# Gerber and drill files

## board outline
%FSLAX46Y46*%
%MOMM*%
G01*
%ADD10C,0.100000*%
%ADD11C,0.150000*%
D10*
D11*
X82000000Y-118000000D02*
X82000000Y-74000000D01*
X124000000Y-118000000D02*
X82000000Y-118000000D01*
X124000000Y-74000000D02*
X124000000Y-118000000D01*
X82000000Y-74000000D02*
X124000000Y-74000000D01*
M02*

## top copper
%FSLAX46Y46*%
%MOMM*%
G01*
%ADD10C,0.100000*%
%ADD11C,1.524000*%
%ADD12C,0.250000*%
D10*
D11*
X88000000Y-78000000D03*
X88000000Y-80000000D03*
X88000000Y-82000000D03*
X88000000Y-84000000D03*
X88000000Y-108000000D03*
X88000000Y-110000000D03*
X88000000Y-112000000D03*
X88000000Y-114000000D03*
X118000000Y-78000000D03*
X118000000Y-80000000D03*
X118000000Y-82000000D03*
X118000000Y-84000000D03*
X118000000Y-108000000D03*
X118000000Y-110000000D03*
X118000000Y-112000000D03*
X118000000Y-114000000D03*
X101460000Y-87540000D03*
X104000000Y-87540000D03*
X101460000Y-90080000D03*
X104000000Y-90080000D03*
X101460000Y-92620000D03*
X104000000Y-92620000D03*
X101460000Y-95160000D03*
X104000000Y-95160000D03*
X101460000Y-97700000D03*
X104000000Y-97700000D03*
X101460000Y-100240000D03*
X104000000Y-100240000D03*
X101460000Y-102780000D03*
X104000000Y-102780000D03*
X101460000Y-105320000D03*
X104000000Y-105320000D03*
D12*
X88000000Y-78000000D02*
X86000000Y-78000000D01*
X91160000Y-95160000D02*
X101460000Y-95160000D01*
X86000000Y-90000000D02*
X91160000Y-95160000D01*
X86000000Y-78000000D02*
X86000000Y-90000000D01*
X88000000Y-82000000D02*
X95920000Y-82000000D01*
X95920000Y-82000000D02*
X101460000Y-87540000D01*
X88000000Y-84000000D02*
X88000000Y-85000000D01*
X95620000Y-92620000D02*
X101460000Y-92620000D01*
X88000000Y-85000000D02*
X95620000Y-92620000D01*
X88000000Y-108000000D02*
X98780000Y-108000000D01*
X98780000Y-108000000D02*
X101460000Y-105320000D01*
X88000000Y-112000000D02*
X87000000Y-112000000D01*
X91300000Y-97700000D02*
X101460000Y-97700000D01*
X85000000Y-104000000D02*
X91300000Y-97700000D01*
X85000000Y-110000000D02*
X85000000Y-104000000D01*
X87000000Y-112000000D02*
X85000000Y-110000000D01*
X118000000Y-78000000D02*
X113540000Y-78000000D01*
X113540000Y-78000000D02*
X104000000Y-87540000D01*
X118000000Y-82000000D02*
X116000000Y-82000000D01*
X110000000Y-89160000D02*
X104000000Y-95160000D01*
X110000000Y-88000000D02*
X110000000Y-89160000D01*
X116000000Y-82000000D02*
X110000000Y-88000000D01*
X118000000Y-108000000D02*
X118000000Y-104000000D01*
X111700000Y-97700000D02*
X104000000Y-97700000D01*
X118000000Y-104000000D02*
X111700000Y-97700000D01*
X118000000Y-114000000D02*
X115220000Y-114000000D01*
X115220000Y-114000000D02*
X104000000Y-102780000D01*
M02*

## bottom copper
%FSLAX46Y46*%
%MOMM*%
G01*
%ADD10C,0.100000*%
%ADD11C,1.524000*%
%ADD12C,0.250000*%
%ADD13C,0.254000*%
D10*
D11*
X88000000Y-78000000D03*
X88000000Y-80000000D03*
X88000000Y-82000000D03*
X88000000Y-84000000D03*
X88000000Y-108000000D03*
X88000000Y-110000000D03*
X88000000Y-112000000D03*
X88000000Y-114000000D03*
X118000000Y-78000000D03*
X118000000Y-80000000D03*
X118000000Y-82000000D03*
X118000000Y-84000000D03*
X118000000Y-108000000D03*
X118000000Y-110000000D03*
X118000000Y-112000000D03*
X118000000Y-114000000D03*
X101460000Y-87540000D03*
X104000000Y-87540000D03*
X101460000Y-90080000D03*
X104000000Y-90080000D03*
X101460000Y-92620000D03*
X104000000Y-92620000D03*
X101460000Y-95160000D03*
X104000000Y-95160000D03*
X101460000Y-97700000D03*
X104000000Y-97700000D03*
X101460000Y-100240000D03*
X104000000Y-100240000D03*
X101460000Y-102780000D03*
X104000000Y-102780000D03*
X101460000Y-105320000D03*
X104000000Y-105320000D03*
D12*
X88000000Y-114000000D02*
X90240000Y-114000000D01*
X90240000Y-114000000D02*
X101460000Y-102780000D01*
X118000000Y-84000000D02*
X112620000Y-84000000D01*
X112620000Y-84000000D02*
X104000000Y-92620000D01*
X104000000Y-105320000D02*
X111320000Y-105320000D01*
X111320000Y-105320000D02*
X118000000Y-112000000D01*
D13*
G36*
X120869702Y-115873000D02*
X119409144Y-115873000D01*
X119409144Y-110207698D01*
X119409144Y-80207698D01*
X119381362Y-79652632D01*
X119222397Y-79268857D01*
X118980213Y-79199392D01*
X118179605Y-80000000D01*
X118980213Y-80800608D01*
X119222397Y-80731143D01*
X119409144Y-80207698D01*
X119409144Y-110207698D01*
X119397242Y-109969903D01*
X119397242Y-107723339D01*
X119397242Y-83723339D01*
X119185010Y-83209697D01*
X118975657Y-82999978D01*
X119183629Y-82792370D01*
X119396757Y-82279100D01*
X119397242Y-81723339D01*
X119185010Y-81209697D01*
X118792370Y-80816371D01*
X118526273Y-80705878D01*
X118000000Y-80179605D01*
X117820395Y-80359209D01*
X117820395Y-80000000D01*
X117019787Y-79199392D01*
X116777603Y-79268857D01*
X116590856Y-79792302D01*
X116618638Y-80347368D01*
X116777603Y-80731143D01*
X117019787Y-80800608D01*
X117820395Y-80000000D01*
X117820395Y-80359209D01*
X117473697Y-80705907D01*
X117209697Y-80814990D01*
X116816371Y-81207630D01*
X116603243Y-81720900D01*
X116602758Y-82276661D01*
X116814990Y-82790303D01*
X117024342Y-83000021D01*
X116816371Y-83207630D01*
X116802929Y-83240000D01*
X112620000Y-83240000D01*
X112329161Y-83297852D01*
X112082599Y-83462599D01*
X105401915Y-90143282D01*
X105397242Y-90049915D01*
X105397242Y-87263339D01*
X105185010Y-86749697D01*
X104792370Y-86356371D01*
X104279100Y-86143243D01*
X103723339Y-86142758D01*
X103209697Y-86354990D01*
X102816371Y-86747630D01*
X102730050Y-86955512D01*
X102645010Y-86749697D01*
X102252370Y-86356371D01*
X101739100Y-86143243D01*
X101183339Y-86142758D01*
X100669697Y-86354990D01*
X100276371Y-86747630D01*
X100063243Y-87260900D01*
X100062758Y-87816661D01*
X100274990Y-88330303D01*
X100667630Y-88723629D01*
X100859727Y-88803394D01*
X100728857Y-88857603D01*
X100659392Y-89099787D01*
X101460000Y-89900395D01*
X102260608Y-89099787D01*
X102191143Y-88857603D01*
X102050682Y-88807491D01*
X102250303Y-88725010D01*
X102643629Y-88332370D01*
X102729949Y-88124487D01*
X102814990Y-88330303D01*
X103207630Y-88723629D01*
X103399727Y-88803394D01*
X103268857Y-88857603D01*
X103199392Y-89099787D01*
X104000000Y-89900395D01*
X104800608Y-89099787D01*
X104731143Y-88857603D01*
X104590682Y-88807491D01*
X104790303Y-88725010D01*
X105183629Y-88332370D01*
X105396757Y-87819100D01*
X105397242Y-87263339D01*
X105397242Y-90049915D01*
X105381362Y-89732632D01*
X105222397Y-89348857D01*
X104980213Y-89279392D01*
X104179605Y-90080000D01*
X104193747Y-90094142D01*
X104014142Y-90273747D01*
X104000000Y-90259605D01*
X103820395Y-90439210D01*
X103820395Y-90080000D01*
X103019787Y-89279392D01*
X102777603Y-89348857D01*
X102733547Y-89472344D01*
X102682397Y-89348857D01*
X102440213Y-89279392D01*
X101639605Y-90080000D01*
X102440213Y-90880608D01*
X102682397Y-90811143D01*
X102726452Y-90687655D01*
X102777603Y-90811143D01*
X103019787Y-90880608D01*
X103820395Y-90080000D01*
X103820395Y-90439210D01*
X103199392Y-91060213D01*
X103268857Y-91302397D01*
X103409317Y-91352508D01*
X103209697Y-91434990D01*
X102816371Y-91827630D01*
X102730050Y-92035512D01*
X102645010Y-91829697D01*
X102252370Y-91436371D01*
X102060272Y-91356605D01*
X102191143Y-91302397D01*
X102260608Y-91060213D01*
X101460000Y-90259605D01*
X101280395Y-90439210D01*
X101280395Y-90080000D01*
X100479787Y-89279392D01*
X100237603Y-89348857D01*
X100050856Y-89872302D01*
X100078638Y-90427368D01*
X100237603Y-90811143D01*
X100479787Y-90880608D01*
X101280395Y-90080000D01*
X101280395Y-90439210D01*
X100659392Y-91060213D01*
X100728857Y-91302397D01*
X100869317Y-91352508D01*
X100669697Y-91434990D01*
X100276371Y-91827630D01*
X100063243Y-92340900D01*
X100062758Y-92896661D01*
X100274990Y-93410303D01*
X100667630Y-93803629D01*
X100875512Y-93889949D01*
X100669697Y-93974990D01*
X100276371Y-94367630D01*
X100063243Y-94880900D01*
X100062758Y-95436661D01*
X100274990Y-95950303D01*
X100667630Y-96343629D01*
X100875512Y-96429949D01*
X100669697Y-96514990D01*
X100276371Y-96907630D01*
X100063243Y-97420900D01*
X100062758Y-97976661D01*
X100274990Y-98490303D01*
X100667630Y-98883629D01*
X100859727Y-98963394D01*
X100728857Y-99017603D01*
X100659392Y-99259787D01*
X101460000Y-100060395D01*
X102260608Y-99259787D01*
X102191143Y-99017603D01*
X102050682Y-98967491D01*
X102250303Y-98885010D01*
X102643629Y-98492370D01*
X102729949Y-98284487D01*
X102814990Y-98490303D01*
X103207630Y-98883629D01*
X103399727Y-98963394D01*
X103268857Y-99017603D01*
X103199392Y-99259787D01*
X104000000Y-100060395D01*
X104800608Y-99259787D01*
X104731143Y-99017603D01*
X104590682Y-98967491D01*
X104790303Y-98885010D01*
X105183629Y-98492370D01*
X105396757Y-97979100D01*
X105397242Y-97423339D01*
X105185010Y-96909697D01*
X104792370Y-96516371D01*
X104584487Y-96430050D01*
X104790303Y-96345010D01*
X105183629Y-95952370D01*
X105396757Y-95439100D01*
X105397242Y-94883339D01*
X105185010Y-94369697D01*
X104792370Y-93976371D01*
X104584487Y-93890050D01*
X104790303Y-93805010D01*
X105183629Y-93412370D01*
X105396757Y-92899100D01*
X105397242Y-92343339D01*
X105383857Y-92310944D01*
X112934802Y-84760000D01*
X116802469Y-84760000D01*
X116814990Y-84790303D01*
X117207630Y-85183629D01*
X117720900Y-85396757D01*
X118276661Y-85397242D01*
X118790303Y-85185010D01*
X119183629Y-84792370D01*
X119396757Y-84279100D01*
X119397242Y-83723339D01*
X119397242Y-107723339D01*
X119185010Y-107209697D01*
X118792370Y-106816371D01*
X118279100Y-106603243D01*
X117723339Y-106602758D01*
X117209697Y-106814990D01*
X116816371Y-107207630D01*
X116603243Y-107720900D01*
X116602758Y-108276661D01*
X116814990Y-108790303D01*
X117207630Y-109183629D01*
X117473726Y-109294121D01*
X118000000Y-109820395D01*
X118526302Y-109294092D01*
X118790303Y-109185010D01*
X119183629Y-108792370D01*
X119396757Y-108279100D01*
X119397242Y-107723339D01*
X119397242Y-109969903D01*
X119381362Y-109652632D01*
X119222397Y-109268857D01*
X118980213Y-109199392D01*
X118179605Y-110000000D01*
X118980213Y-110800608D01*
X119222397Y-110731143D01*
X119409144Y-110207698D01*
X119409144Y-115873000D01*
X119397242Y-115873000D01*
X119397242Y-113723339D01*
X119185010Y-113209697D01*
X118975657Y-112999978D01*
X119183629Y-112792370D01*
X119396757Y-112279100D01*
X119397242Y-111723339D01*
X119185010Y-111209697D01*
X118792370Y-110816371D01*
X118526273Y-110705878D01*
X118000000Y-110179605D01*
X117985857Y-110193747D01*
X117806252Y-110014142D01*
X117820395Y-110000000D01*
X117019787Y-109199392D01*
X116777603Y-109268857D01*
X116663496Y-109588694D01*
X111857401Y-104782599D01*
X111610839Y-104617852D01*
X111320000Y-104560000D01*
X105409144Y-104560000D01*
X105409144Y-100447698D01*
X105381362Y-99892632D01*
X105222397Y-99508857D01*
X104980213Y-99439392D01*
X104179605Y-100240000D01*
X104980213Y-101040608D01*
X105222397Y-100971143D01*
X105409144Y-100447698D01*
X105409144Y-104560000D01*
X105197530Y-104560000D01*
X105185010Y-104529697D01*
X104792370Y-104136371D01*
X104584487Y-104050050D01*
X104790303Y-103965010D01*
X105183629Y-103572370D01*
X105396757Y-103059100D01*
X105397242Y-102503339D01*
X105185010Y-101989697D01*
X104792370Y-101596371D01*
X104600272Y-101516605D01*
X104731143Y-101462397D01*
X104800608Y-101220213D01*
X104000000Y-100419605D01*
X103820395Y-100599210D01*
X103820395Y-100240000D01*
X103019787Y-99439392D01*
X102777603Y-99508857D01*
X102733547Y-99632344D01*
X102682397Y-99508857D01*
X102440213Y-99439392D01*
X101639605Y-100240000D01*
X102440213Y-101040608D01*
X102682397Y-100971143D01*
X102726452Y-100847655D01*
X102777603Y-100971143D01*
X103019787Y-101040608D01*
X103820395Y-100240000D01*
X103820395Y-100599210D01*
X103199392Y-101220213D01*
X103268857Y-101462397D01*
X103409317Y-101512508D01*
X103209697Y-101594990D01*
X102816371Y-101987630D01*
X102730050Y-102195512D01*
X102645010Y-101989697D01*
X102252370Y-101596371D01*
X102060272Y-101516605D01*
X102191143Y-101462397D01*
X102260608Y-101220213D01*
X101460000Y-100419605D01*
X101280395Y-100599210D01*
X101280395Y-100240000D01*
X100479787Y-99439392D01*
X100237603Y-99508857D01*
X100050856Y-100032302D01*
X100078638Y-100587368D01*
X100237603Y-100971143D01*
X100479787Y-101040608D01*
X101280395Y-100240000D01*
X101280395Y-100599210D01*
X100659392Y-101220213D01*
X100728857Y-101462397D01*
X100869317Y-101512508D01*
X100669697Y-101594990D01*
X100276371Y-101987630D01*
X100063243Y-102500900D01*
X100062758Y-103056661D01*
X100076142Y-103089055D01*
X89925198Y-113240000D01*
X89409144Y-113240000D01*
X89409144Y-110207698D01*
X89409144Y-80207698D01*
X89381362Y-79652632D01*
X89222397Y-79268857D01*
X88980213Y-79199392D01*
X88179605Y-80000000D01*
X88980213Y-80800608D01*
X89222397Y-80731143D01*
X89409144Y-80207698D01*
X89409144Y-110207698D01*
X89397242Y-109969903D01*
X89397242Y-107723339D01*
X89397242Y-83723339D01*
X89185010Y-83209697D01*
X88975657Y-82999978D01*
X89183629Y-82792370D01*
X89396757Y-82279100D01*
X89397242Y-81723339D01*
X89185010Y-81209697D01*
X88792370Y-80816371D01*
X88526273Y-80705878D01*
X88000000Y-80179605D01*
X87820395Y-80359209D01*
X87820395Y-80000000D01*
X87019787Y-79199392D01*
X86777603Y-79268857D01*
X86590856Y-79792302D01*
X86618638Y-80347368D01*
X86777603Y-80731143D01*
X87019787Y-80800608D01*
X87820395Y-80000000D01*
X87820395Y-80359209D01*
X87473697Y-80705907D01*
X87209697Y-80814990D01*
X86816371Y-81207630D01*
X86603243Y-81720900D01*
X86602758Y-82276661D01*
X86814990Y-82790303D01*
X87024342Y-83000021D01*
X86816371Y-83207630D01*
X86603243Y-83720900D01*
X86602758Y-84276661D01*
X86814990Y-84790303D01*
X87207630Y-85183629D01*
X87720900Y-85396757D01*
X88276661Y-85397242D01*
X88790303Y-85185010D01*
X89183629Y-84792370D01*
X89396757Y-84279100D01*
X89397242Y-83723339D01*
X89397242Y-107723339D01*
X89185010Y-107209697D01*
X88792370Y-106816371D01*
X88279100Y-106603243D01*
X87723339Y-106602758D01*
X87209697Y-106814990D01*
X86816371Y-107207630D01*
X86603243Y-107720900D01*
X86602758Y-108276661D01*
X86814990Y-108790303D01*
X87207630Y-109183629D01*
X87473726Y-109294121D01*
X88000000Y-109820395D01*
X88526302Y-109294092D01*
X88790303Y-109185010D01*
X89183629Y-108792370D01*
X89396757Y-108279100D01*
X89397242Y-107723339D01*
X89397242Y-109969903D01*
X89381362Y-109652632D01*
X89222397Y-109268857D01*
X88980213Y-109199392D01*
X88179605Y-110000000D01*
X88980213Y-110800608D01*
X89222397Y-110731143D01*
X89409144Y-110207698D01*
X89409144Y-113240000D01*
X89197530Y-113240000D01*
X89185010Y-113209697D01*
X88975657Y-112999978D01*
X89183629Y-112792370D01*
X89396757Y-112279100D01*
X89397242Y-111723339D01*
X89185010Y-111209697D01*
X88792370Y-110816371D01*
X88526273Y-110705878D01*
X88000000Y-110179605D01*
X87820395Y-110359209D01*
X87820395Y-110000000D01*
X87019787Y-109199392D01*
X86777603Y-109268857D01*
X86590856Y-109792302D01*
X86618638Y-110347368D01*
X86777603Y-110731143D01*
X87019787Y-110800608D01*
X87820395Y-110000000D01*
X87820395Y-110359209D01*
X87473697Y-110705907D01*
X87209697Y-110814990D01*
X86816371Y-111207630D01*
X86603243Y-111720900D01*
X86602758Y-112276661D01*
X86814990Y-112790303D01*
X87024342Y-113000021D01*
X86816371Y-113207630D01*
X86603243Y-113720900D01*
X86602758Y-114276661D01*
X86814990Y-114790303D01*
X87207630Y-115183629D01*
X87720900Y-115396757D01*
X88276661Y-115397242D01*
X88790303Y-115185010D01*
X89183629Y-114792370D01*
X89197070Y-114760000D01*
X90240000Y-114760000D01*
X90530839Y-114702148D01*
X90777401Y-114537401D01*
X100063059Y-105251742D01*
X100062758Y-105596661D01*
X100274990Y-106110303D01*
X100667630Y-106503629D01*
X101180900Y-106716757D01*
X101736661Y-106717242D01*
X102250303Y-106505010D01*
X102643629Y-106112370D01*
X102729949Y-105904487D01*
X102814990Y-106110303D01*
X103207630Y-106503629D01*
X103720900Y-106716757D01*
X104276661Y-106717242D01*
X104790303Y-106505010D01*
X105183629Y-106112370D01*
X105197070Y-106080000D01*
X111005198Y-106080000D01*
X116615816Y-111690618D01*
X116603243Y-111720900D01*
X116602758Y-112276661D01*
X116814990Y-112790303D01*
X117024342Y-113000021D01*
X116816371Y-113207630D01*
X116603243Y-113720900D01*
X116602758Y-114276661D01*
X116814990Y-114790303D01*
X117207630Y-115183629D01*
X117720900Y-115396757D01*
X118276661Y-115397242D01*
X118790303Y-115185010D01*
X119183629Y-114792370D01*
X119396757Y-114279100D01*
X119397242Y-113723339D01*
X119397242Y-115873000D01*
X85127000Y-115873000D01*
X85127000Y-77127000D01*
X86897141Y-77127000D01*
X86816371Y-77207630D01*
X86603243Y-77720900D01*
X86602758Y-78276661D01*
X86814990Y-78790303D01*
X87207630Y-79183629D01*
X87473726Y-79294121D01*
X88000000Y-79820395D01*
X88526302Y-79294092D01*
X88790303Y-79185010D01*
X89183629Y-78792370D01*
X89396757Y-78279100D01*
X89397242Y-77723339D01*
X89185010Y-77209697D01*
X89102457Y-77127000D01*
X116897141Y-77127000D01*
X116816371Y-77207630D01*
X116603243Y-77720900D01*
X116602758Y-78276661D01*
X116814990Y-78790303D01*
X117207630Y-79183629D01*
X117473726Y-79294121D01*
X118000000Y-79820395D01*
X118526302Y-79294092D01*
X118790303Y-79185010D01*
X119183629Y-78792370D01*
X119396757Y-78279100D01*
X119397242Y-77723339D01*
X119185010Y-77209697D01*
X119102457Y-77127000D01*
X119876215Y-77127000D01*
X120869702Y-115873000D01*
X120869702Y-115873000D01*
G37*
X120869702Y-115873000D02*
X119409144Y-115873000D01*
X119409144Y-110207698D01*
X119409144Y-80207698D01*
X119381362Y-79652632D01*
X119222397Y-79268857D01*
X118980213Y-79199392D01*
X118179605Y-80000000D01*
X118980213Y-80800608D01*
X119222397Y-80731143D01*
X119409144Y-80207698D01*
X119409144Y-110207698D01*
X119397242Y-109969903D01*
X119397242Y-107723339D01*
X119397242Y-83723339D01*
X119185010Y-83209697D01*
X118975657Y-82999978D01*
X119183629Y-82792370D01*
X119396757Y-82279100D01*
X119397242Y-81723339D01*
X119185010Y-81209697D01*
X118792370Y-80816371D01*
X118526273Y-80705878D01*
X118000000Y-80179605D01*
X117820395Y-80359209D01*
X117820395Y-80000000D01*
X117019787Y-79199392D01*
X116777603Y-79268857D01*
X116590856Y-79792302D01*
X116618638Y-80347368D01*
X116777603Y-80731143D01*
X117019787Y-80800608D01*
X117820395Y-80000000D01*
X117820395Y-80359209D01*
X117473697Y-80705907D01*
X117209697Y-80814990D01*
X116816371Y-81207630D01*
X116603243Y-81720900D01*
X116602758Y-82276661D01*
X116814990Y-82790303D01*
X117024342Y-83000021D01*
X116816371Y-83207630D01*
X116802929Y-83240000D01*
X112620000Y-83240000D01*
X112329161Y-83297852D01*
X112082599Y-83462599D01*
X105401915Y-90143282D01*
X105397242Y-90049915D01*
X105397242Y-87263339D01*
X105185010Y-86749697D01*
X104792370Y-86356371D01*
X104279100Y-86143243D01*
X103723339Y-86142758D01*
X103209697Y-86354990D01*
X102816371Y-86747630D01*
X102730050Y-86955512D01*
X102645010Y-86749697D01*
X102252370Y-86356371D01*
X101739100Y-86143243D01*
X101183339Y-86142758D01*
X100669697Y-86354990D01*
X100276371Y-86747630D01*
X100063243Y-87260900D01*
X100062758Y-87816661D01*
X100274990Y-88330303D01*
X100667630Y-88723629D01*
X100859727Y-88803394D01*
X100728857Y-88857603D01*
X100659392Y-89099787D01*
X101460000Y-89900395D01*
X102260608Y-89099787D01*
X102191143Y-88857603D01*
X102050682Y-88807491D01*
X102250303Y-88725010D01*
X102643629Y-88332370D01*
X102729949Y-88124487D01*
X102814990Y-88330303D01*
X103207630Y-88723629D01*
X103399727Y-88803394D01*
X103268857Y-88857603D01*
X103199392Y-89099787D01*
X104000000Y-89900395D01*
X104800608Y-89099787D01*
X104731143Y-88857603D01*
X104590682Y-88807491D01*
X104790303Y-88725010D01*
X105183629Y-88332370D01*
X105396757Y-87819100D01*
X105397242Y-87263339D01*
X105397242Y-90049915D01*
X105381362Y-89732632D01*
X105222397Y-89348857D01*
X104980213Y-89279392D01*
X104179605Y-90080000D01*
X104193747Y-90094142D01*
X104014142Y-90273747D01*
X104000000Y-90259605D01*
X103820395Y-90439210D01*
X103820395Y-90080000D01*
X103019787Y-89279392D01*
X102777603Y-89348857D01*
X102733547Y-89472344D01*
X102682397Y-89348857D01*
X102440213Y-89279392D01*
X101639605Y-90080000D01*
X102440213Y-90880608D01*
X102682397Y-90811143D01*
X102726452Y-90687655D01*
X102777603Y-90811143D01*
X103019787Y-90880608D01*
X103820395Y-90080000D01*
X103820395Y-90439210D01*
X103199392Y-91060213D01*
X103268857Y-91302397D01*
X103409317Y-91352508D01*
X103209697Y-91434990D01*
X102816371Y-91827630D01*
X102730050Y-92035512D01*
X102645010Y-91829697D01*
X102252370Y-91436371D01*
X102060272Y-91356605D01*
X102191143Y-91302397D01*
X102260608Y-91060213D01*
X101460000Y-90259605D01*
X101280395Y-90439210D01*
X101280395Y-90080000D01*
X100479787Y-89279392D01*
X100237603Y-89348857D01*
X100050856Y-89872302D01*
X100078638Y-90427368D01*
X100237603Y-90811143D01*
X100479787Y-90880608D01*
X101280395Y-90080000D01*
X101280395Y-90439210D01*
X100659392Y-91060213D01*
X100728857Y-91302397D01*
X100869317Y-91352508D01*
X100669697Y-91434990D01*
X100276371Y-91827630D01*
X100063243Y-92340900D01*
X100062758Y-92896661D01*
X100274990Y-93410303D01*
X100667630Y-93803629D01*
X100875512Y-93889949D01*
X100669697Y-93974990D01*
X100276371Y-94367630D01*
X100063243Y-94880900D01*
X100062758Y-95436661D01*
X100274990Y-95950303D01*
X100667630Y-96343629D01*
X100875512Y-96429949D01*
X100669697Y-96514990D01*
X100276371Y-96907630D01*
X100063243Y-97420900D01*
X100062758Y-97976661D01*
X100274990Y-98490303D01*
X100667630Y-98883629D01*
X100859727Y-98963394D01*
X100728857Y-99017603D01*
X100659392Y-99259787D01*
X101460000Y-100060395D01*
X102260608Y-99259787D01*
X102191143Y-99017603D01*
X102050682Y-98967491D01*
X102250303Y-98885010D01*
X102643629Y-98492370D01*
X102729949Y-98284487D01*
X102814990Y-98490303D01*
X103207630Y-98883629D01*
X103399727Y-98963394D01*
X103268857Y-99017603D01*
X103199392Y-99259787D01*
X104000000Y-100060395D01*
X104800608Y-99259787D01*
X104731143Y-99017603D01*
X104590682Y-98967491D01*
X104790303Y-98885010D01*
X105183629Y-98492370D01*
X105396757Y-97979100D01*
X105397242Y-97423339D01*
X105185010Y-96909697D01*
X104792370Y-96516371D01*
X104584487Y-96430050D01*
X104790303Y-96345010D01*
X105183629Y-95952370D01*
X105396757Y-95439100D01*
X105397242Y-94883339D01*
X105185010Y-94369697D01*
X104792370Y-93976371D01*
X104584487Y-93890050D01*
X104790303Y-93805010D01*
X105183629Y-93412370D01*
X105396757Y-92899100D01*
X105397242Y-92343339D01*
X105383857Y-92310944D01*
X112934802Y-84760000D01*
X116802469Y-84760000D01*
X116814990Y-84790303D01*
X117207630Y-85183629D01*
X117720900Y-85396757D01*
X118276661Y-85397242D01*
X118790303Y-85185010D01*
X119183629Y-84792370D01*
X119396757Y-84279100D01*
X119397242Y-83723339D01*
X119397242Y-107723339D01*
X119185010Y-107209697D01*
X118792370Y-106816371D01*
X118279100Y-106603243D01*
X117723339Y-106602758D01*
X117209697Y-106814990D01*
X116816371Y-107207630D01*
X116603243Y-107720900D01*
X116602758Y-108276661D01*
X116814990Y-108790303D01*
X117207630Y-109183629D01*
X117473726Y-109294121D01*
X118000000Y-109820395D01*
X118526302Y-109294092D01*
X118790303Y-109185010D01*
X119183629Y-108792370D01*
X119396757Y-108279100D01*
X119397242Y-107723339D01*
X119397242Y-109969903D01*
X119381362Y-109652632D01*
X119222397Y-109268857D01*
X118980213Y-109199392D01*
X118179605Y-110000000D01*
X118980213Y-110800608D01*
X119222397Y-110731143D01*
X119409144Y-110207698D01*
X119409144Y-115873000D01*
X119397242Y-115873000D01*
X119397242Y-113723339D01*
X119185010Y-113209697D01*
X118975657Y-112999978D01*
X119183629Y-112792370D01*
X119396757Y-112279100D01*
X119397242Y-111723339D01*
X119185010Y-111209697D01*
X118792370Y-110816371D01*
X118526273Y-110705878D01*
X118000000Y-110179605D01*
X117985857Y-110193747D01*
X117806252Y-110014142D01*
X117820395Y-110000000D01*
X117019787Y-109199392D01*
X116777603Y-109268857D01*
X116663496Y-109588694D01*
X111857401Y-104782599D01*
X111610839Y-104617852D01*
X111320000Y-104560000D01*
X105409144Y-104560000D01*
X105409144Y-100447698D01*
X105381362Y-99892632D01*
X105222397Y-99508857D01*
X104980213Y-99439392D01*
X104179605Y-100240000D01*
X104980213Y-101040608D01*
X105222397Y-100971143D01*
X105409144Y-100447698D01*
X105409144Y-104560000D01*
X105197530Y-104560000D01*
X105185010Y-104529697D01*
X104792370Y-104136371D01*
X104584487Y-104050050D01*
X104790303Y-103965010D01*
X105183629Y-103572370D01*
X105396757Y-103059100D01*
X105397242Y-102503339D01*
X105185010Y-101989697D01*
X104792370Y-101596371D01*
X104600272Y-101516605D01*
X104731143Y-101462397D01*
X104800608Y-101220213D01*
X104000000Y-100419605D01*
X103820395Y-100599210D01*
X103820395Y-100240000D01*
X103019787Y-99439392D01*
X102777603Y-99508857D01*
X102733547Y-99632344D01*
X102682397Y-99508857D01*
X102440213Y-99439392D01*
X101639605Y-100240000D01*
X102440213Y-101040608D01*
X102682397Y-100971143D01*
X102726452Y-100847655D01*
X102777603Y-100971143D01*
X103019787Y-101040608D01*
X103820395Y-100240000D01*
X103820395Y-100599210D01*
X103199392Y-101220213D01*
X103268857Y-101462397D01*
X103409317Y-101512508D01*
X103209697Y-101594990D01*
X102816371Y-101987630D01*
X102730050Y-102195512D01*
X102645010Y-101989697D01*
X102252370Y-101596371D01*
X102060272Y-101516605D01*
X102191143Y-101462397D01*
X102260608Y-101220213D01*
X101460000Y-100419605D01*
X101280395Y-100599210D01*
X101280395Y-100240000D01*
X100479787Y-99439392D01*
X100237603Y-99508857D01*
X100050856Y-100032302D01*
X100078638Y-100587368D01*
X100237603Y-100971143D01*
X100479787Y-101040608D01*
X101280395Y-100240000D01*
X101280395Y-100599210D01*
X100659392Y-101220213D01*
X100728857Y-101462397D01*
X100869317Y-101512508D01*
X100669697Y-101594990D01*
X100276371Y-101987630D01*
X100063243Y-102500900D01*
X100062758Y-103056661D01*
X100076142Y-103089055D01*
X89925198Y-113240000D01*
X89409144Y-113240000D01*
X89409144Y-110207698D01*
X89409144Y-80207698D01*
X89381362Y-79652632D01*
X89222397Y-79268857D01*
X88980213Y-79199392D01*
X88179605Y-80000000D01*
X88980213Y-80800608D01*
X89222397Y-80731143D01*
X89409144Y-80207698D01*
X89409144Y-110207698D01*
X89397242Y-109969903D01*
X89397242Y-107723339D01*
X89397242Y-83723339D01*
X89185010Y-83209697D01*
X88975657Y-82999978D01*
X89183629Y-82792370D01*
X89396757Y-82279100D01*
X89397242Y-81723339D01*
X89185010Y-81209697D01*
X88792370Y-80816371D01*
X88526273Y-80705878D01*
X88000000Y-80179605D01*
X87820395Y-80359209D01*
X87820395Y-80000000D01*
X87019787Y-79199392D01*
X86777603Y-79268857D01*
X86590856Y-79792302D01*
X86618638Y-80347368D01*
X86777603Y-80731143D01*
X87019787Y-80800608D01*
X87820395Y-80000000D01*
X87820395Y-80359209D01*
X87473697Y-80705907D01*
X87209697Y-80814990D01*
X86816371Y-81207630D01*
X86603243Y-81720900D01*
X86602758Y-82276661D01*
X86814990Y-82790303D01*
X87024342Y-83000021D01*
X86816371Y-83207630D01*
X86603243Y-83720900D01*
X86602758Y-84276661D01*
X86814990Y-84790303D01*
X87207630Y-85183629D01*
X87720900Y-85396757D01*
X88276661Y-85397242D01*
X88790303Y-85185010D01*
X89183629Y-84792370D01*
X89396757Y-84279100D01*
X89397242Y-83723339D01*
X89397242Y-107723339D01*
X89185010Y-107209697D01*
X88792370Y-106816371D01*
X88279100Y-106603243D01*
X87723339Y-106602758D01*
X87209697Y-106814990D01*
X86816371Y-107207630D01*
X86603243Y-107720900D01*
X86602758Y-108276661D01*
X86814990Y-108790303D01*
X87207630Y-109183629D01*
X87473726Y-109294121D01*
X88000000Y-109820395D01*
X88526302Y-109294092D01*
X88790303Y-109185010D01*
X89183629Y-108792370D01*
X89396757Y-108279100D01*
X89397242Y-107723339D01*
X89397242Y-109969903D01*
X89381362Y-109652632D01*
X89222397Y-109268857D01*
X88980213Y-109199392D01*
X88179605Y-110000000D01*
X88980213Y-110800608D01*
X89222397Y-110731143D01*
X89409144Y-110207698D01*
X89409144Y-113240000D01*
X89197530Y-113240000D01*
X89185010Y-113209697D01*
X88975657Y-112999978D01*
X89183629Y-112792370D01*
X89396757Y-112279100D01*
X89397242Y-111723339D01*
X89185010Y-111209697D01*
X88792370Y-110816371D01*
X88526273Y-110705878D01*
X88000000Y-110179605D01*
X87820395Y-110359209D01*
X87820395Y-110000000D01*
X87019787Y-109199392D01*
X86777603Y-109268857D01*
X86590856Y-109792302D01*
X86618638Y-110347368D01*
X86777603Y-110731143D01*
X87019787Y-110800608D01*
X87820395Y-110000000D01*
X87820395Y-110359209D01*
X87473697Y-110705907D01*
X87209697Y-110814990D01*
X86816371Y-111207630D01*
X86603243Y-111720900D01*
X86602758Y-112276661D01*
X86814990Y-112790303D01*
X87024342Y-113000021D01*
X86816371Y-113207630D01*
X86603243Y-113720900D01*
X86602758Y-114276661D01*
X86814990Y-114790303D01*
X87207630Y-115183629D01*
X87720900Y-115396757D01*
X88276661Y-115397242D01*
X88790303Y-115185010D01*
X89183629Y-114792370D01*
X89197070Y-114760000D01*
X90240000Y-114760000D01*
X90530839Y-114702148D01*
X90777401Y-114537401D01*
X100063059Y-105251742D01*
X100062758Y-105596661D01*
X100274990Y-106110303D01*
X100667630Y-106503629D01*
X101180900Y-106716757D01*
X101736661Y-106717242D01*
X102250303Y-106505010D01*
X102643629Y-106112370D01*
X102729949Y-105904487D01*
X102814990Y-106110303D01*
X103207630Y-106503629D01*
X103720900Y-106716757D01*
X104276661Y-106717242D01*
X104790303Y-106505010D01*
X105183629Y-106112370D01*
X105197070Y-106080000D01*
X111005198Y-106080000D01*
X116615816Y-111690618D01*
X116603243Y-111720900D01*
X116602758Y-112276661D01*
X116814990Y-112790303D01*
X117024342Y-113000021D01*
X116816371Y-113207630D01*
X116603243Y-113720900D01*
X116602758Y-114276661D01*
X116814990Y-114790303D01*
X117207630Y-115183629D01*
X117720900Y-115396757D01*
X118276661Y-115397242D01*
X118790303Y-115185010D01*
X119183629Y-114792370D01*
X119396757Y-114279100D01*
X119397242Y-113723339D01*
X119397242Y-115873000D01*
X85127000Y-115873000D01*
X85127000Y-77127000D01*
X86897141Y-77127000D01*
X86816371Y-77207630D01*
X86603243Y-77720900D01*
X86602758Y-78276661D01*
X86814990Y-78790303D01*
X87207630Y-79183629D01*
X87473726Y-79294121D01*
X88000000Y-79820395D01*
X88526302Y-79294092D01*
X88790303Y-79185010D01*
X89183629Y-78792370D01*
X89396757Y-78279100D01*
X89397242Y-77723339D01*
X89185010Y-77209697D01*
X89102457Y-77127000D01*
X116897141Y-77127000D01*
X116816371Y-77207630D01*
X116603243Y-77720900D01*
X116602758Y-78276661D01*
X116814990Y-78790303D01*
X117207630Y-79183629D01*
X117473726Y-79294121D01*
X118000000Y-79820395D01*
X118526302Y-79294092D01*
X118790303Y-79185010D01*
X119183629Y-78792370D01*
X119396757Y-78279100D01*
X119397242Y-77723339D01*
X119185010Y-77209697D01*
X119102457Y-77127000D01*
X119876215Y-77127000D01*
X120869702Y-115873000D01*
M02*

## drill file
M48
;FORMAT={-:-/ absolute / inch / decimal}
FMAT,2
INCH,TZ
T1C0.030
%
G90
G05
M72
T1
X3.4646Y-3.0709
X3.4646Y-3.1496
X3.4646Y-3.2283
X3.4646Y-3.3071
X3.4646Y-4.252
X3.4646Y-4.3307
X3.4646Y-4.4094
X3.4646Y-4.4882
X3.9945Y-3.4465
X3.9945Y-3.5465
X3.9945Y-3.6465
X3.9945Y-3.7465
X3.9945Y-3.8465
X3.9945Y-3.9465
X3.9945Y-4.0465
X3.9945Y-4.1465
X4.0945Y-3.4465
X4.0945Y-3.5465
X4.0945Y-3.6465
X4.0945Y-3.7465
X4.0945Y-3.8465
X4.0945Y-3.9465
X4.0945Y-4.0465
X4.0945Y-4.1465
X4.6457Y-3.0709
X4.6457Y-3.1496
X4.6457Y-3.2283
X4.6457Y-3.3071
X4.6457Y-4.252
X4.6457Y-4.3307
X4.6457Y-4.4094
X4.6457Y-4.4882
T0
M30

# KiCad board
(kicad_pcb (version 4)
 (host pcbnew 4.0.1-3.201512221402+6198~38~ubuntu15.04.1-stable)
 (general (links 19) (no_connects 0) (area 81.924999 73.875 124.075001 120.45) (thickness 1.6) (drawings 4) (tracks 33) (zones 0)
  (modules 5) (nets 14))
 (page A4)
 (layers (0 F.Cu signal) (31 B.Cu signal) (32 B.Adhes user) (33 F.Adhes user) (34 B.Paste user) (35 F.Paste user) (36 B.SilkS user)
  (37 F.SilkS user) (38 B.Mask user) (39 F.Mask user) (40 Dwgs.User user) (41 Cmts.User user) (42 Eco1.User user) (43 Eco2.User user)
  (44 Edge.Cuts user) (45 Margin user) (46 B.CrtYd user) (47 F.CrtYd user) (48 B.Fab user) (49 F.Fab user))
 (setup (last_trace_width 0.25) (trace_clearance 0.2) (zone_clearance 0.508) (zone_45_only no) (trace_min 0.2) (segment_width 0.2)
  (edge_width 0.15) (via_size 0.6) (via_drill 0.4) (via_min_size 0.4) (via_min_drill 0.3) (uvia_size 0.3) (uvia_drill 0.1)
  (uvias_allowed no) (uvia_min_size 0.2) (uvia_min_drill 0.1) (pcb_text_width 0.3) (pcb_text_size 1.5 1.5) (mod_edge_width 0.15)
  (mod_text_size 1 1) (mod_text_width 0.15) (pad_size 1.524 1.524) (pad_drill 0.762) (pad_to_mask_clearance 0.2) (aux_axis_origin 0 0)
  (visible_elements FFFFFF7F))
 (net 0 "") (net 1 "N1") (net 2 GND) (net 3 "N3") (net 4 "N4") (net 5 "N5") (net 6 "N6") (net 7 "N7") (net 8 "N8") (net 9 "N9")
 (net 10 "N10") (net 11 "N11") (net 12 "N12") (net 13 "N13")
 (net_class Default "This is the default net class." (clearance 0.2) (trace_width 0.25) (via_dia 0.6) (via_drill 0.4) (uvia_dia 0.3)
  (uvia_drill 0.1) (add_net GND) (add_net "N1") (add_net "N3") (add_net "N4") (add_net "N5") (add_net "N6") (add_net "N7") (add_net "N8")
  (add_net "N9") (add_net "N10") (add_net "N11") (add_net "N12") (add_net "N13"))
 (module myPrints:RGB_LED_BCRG (layer F.Cu) (at 90 90)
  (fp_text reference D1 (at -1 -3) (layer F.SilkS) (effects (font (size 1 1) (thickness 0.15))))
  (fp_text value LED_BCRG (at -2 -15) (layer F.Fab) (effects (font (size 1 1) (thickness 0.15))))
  (pad 1 thru_hole circle (at -2 -12) (size 1.524 1.524) (drill 0.762) (layers *.Cu *.Mask F.SilkS) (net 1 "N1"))
  (pad 2 thru_hole circle (at -2 -10) (size 1.524 1.524) (drill 0.762) (layers *.Cu *.Mask F.SilkS) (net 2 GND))
  (pad 3 thru_hole circle (at -2 -8) (size 1.524 1.524) (drill 0.762) (layers *.Cu *.Mask F.SilkS) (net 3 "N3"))
  (pad 4 thru_hole circle (at -2 -6) (size 1.524 1.524) (drill 0.762) (layers *.Cu *.Mask F.SilkS) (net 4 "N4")))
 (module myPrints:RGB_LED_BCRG (layer F.Cu) (at 90 120)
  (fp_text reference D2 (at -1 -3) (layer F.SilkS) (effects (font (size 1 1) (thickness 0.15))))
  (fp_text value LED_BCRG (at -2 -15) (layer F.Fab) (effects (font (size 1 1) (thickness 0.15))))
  (pad 1 thru_hole circle (at -2 -12) (size 1.524 1.524) (drill 0.762) (layers *.Cu *.Mask F.SilkS) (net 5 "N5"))
  (pad 2 thru_hole circle (at -2 -10) (size 1.524 1.524) (drill 0.762) (layers *.Cu *.Mask F.SilkS) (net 2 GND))
  (pad 3 thru_hole circle (at -2 -8) (size 1.524 1.524) (drill 0.762) (layers *.Cu *.Mask F.SilkS) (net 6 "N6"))
  (pad 4 thru_hole circle (at -2 -6) (size 1.524 1.524) (drill 0.762) (layers *.Cu *.Mask F.SilkS) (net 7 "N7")))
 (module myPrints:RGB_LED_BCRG (layer F.Cu) (at 120 90)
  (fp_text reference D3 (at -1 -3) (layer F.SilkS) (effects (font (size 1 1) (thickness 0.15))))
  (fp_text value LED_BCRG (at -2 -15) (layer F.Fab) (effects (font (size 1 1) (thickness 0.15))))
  (pad 1 thru_hole circle (at -2 -12) (size 1.524 1.524) (drill 0.762) (layers *.Cu *.Mask F.SilkS) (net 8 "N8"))
  (pad 2 thru_hole circle (at -2 -10) (size 1.524 1.524) (drill 0.762) (layers *.Cu *.Mask F.SilkS) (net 2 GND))
  (pad 3 thru_hole circle (at -2 -8) (size 1.524 1.524) (drill 0.762) (layers *.Cu *.Mask F.SilkS) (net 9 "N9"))
  (pad 4 thru_hole circle (at -2 -6) (size 1.524 1.524) (drill 0.762) (layers *.Cu *.Mask F.SilkS) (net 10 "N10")))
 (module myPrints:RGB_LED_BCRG (layer F.Cu) (at 120 120)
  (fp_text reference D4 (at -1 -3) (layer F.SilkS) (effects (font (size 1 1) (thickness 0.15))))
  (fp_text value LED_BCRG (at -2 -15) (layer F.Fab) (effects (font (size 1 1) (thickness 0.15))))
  (pad 1 thru_hole circle (at -2 -12) (size 1.524 1.524) (drill 0.762) (layers *.Cu *.Mask F.SilkS) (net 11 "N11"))
  (pad 2 thru_hole circle (at -2 -10) (size 1.524 1.524) (drill 0.762) (layers *.Cu *.Mask F.SilkS) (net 2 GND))
  (pad 3 thru_hole circle (at -2 -8) (size 1.524 1.524) (drill 0.762) (layers *.Cu *.Mask F.SilkS) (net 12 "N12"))
  (pad 4 thru_hole circle (at -2 -6) (size 1.524 1.524) (drill 0.762) (layers *.Cu *.Mask F.SilkS) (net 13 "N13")))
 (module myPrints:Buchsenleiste (layer F.Cu) (at 104 85)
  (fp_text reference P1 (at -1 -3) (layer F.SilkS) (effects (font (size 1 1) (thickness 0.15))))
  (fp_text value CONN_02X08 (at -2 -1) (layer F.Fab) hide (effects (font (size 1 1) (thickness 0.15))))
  (pad 1 thru_hole circle (at -2.54 2.54) (size 1.524 1.524) (drill 0.762) (layers *.Cu *.Mask F.SilkS) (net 3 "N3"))
  (pad 2 thru_hole circle (at 0 2.54) (size 1.524 1.524) (drill 0.762) (layers *.Cu *.Mask F.SilkS) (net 8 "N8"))
  (pad 3 thru_hole circle (at -2.54 5.08) (size 1.524 1.524) (drill 0.762) (layers *.Cu *.Mask F.SilkS) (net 2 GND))
  (pad 4 thru_hole circle (at 0 5.08) (size 1.524 1.524) (drill 0.762) (layers *.Cu *.Mask F.SilkS) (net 2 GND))
  (pad 5 thru_hole circle (at -2.54 7.62) (size 1.524 1.524) (drill 0.762) (layers *.Cu *.Mask F.SilkS) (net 4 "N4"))
  (pad 6 thru_hole circle (at 0 7.62) (size 1.524 1.524) (drill 0.762) (layers *.Cu *.Mask F.SilkS) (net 10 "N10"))
  (pad 7 thru_hole circle (at -2.54 10.16) (size 1.524 1.524) (drill 0.762) (layers *.Cu *.Mask F.SilkS) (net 1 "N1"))
  (pad 8 thru_hole circle (at 0 10.16) (size 1.524 1.524) (drill 0.762) (layers *.Cu *.Mask F.SilkS) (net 9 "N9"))
  (pad 9 thru_hole circle (at -2.54 12.7) (size 1.524 1.524) (drill 0.762) (layers *.Cu *.Mask F.SilkS) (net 6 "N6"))
  (pad 10 thru_hole circle (at 0 12.7) (size 1.524 1.524) (drill 0.762) (layers *.Cu *.Mask F.SilkS) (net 11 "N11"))
  (pad 11 thru_hole circle (at -2.54 15.24) (size 1.524 1.524) (drill 0.762) (layers *.Cu *.Mask F.SilkS) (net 2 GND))
  (pad 12 thru_hole circle (at 0 15.24) (size 1.524 1.524) (drill 0.762) (layers *.Cu *.Mask F.SilkS) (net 2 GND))
  (pad 13 thru_hole circle (at -2.54 17.78) (size 1.524 1.524) (drill 0.762) (layers *.Cu *.Mask F.SilkS) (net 7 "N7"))
  (pad 14 thru_hole circle (at 0 17.78) (size 1.524 1.524) (drill 0.762) (layers *.Cu *.Mask F.SilkS) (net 13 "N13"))
  (pad 15 thru_hole circle (at -2.54 20.32) (size 1.524 1.524) (drill 0.762) (layers *.Cu *.Mask F.SilkS) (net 5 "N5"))
  (pad 16 thru_hole circle (at 0 20.32) (size 1.524 1.524) (drill 0.762) (layers *.Cu *.Mask F.SilkS) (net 12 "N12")))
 (gr_line (start 82 118) (end 82 74) (angle 90) (layer Edge.Cuts) (width 0.15))
 (gr_line (start 124 118) (end 82 118) (angle 90) (layer Edge.Cuts) (width 0.15))
 (gr_line (start 124 74) (end 124 118) (angle 90) (layer Edge.Cuts) (width 0.15))
 (gr_line (start 82 74) (end 124 74) (angle 90) (layer Edge.Cuts) (width 0.15))
 (segment (start 88 78) (end 86 78) (width 0.25) (layer F.Cu) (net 1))
 (segment (start 91.16 95.16) (end 101.46 95.16) (width 0.25) (layer F.Cu) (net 1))
 (segment (start 86 90) (end 91.16 95.16) (width 0.25) (layer F.Cu) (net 1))
 (segment (start 86 78) (end 86 90) (width 0.25) (layer F.Cu) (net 1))
 (segment (start 88 82) (end 95.92 82) (width 0.25) (layer F.Cu) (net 3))
 (segment (start 95.92 82) (end 101.46 87.54) (width 0.25) (layer F.Cu) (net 3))
 (segment (start 88 84) (end 88 85) (width 0.25) (layer F.Cu) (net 4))
 (segment (start 95.62 92.62) (end 101.46 92.62) (width 0.25) (layer F.Cu) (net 4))
 (segment (start 88 85) (end 95.62 92.62) (width 0.25) (layer F.Cu) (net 4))
 (segment (start 88 108) (end 98.78 108) (width 0.25) (layer F.Cu) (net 5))
 (segment (start 98.78 108) (end 101.46 105.32) (width 0.25) (layer F.Cu) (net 5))
 (segment (start 88 112) (end 87 112) (width 0.25) (layer F.Cu) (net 6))
 (segment (start 91.3 97.7) (end 101.46 97.7) (width 0.25) (layer F.Cu) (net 6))
 (segment (start 85 104) (end 91.3 97.7) (width 0.25) (layer F.Cu) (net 6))
 (segment (start 85 110) (end 85 104) (width 0.25) (layer F.Cu) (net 6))
 (segment (start 87 112) (end 85 110) (width 0.25) (layer F.Cu) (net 6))
 (segment (start 88 114) (end 90.24 114) (width 0.25) (layer B.Cu) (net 7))
 (segment (start 90.24 114) (end 101.46 102.78) (width 0.25) (layer B.Cu) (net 7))
 (segment (start 118 78) (end 113.54 78) (width 0.25) (layer F.Cu) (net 8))
 (segment (start 113.54 78) (end 104 87.54) (width 0.25) (layer F.Cu) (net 8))
 (segment (start 118 82) (end 116 82) (width 0.25) (layer F.Cu) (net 9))
 (segment (start 110 89.16) (end 104 95.16) (width 0.25) (layer F.Cu) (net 9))
 (segment (start 110 88) (end 110 89.16) (width 0.25) (layer F.Cu) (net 9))
 (segment (start 116 82) (end 110 88) (width 0.25) (layer F.Cu) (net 9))
 (segment (start 118 84) (end 112.62 84) (width 0.25) (layer B.Cu) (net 10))
 (segment (start 112.62 84) (end 104 92.62) (width 0.25) (layer B.Cu) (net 10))
 (segment (start 118 108) (end 118 104) (width 0.25) (layer F.Cu) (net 11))
 (segment (start 111.7 97.7) (end 104 97.7) (width 0.25) (layer F.Cu) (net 11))
 (segment (start 118 104) (end 111.7 97.7) (width 0.25) (layer F.Cu) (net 11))
 (segment (start 104 105.32) (end 111.32 105.32) (width 0.25) (layer B.Cu) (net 12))
 (segment (start 111.32 105.32) (end 118 112) (width 0.25) (layer B.Cu) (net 12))
 (segment (start 118 114) (end 115.22 114) (width 0.25) (layer F.Cu) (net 13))
 (segment (start 115.22 114) (end 104 102.78) (width 0.25) (layer F.Cu) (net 13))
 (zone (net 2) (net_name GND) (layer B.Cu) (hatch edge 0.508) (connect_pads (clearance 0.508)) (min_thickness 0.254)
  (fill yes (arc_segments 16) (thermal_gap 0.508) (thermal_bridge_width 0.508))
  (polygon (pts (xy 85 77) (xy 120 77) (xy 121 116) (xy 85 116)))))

